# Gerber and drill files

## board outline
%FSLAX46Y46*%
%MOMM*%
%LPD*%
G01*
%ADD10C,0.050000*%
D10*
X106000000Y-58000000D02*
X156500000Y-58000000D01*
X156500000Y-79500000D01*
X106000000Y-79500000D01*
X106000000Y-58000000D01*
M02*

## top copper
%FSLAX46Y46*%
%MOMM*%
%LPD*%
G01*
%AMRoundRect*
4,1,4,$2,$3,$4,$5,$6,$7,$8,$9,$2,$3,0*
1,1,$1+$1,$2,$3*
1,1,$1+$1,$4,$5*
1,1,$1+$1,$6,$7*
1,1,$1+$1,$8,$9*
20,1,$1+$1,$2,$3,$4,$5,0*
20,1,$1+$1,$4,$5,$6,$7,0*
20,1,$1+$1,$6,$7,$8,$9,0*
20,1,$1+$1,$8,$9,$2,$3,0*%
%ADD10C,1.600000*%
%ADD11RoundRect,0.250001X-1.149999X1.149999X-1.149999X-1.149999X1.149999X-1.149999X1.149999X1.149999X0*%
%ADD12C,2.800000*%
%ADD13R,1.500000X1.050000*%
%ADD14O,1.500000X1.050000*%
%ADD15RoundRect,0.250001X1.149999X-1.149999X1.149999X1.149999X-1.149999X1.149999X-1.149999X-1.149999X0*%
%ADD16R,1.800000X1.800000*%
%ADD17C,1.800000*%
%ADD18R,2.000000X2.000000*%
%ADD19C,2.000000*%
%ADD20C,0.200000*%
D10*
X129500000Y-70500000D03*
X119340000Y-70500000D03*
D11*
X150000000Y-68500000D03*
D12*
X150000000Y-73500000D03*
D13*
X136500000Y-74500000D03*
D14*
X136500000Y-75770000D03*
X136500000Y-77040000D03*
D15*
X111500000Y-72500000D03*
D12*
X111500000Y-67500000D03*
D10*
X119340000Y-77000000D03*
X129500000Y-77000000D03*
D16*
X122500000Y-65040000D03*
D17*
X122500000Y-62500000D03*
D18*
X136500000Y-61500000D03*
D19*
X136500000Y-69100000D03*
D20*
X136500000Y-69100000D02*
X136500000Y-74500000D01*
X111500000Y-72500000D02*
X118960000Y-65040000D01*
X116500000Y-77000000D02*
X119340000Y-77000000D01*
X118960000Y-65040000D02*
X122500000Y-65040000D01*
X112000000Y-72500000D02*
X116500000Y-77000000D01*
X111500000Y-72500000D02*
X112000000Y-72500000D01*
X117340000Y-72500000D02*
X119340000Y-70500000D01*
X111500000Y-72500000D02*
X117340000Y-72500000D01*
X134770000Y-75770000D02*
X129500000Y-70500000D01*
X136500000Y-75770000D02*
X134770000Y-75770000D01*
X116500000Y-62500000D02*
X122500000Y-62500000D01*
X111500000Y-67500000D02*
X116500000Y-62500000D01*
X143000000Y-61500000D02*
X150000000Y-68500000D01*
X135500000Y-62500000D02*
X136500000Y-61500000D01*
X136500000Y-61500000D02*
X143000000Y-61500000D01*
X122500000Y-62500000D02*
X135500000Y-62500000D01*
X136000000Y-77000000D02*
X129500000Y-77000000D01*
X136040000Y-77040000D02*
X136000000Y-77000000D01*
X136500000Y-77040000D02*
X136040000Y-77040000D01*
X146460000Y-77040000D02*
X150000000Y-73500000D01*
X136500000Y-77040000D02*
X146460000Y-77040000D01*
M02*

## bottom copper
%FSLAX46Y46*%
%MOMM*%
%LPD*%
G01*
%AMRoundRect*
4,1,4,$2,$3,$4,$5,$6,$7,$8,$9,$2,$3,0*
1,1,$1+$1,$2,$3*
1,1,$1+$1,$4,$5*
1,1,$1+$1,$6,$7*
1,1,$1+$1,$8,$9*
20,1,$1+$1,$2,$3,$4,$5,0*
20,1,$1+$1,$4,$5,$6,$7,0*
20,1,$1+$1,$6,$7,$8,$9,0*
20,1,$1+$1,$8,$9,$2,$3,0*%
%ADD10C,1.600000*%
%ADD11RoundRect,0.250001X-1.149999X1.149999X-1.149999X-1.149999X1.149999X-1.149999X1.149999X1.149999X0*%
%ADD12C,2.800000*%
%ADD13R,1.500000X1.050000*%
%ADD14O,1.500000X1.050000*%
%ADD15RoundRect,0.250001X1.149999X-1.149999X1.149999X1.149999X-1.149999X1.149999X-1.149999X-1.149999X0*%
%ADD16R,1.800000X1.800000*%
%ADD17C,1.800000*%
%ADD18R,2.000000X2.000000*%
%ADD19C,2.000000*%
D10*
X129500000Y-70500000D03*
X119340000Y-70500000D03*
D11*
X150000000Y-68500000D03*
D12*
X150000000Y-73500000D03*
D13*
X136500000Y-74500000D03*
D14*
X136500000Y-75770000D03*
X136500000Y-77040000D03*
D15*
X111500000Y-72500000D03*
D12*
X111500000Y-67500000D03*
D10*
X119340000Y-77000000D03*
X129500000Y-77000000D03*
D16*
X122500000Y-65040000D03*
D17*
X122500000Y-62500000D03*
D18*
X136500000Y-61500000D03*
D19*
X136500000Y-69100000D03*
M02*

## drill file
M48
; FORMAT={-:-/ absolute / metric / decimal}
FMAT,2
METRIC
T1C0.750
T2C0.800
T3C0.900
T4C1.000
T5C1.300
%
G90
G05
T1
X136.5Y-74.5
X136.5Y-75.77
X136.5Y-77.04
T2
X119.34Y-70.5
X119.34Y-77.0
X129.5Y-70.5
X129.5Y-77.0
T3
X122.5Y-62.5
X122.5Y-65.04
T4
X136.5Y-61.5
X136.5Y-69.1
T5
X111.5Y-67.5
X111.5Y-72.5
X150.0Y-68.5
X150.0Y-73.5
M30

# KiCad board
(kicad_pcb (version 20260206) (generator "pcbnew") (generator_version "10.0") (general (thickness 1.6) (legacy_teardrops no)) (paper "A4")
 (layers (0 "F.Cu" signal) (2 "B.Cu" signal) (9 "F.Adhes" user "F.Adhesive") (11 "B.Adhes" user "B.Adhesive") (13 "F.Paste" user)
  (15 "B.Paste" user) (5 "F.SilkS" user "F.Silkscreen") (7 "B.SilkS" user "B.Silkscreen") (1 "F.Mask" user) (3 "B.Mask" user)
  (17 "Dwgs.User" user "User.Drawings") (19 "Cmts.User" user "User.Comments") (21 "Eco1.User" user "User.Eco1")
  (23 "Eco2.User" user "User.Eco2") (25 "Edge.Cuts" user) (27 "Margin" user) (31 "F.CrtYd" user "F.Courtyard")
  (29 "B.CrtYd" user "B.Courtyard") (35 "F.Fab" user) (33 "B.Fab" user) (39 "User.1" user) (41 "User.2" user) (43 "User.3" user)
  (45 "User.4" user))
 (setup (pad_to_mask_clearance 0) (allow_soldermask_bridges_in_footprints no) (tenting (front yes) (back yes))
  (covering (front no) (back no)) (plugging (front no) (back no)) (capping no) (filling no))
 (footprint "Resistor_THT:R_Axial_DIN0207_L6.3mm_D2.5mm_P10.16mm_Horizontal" (layer "F.Cu") (at 129.5 70.5 180)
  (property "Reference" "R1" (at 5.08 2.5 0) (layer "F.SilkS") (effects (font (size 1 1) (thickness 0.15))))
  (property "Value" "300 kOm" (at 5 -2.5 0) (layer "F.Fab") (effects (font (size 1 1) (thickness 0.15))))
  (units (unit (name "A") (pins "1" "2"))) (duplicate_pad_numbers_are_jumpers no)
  (pad "1" thru_hole circle (at 0 0 180) (size 1.6 1.6) (drill 0.8) (layers "*.Cu" "*.Mask") (remove_unused_layers no) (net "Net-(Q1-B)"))
  (pad "2" thru_hole circle (at 10.16 0 180) (size 1.6 1.6) (drill 0.8) (layers "*.Cu" "*.Mask") (remove_unused_layers no)
   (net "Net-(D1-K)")))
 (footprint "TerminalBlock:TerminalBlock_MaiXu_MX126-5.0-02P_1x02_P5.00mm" (layer "F.Cu") (at 150 68.5 -90)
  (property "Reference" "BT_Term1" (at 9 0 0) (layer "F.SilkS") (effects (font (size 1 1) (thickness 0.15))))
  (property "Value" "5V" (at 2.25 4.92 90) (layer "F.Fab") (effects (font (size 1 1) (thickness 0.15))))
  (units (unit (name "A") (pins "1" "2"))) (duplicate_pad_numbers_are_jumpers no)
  (pad "1" thru_hole roundrect (at 0 0 270) (size 2.8 2.8) (drill 1.3) (layers "*.Cu" "*.Mask") (remove_unused_layers no)
   (roundrect_rratio 0.089286) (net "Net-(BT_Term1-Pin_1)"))
  (pad "2" thru_hole circle (at 5 0 270) (size 2.8 2.8) (drill 1.3) (layers "*.Cu" "*.Mask") (remove_unused_layers no)
   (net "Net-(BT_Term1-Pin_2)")))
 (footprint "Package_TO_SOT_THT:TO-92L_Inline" (layer "F.Cu") (at 136.5 74.5 -90)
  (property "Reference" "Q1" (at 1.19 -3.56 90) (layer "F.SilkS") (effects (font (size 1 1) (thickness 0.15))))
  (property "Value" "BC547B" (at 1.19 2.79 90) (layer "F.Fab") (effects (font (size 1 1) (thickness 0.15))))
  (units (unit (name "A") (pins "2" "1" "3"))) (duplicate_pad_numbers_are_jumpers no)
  (pad "1" thru_hole rect (at 0 0 270) (size 1.05 1.5) (drill 0.75) (layers "*.Cu" "*.Mask") (remove_unused_layers no) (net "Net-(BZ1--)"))
  (pad "2" thru_hole oval (at 1.27 0 270) (size 1.05 1.5) (drill 0.75) (layers "*.Cu" "*.Mask") (remove_unused_layers no) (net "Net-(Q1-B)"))
  (pad "3" thru_hole oval (at 2.54 0 270) (size 1.05 1.5) (drill 0.75) (layers "*.Cu" "*.Mask") (remove_unused_layers no)
   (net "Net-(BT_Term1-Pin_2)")))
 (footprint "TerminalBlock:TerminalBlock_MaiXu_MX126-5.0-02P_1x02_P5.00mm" (layer "F.Cu") (at 111.5 72.5 90)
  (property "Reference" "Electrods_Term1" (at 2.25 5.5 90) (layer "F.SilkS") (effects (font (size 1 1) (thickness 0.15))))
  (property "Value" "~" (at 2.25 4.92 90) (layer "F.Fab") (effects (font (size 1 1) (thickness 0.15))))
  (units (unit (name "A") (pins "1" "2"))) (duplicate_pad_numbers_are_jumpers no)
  (pad "1" thru_hole roundrect (at 0 0 90) (size 2.8 2.8) (drill 1.3) (layers "*.Cu" "*.Mask") (remove_unused_layers no)
   (roundrect_rratio 0.089286) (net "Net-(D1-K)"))
  (pad "2" thru_hole circle (at 5 0 90) (size 2.8 2.8) (drill 1.3) (layers "*.Cu" "*.Mask") (remove_unused_layers no)
   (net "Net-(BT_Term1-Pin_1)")))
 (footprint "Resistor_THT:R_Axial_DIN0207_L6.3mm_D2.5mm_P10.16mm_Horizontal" (layer "F.Cu") (at 119.34 77)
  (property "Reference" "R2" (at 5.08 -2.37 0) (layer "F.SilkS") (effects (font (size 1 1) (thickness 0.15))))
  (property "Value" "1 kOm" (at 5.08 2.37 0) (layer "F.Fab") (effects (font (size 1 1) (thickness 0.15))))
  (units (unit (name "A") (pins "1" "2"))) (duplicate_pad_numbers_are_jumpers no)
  (pad "1" thru_hole circle (at 0 0) (size 1.6 1.6) (drill 0.8) (layers "*.Cu" "*.Mask") (remove_unused_layers no) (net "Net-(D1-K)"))
  (pad "2" thru_hole circle (at 10.16 0) (size 1.6 1.6) (drill 0.8) (layers "*.Cu" "*.Mask") (remove_unused_layers no)
   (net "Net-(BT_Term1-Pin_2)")))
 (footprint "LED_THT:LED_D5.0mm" (layer "F.Cu") (at 122.5 65.04 90)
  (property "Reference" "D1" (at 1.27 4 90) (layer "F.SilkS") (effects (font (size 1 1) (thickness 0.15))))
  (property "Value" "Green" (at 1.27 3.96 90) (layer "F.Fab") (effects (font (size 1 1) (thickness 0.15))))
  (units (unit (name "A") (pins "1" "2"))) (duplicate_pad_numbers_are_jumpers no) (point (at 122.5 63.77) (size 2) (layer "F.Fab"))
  (pad "1" thru_hole rect (at 0 0 90) (size 1.8 1.8) (drill 0.9) (layers "*.Cu" "*.Mask") (remove_unused_layers no) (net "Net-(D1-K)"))
  (pad "2" thru_hole circle (at 2.54 0 90) (size 1.8 1.8) (drill 0.9) (layers "*.Cu" "*.Mask") (remove_unused_layers no)
   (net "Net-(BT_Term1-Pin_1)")))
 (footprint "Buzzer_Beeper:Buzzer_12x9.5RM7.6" (layer "F.Cu") (at 136.5 61.5 -90)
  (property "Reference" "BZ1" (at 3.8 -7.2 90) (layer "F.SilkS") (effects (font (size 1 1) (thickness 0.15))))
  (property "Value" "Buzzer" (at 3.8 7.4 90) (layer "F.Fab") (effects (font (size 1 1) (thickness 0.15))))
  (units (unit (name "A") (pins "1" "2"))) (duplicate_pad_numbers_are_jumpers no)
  (pad "1" thru_hole rect (at 0 0 270) (size 2 2) (drill 1) (layers "*.Cu" "*.Mask") (remove_unused_layers no) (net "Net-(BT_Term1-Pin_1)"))
  (pad "2" thru_hole circle (at 7.6 0 270) (size 2 2) (drill 1) (layers "*.Cu" "*.Mask") (remove_unused_layers no) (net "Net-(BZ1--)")))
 (gr_rect (start 106 58) (end 156.5 79.5) (stroke (width 0.05) (type default)) (fill no) (layer "Edge.Cuts"))
 (segment (start 136.5 69.1) (end 136.5 74.5) (width 0.2) (layer "F.Cu") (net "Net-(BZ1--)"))
 (segment (start 111.5 72.5) (end 118.96 65.04) (width 0.2) (layer "F.Cu") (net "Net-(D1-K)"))
 (segment (start 116.5 77) (end 119.34 77) (width 0.2) (layer "F.Cu") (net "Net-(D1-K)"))
 (segment (start 118.96 65.04) (end 122.5 65.04) (width 0.2) (layer "F.Cu") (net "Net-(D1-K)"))
 (segment (start 112 72.5) (end 116.5 77) (width 0.2) (layer "F.Cu") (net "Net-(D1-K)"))
 (segment (start 111.5 72.5) (end 112 72.5) (width 0.2) (layer "F.Cu") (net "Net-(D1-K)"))
 (segment (start 117.34 72.5) (end 119.34 70.5) (width 0.2) (layer "F.Cu") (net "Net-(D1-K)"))
 (segment (start 111.5 72.5) (end 117.34 72.5) (width 0.2) (layer "F.Cu") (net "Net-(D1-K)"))
 (segment (start 134.77 75.77) (end 129.5 70.5) (width 0.2) (layer "F.Cu") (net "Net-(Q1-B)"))
 (segment (start 136.5 75.77) (end 134.77 75.77) (width 0.2) (layer "F.Cu") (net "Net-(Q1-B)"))
 (segment (start 116.5 62.5) (end 122.5 62.5) (width 0.2) (layer "F.Cu") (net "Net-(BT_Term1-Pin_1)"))
 (segment (start 111.5 67.5) (end 116.5 62.5) (width 0.2) (layer "F.Cu") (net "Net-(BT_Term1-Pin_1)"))
 (segment (start 143 61.5) (end 150 68.5) (width 0.2) (layer "F.Cu") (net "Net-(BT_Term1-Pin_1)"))
 (segment (start 135.5 62.5) (end 136.5 61.5) (width 0.2) (layer "F.Cu") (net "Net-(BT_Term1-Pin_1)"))
 (segment (start 136.5 61.5) (end 143 61.5) (width 0.2) (layer "F.Cu") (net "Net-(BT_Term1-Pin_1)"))
 (segment (start 122.5 62.5) (end 135.5 62.5) (width 0.2) (layer "F.Cu") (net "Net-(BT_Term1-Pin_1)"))
 (segment (start 136 77) (end 129.5 77) (width 0.2) (layer "F.Cu") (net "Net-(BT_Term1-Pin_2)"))
 (segment (start 136.04 77.04) (end 136 77) (width 0.2) (layer "F.Cu") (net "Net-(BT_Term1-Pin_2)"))
 (segment (start 136.5 77.04) (end 136.04 77.04) (width 0.2) (layer "F.Cu") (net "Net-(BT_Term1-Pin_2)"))
 (segment (start 146.46 77.04) (end 150 73.5) (width 0.2) (layer "F.Cu") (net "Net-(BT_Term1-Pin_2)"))
 (segment (start 136.5 77.04) (end 146.46 77.04) (width 0.2) (layer "F.Cu") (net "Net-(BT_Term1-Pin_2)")))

